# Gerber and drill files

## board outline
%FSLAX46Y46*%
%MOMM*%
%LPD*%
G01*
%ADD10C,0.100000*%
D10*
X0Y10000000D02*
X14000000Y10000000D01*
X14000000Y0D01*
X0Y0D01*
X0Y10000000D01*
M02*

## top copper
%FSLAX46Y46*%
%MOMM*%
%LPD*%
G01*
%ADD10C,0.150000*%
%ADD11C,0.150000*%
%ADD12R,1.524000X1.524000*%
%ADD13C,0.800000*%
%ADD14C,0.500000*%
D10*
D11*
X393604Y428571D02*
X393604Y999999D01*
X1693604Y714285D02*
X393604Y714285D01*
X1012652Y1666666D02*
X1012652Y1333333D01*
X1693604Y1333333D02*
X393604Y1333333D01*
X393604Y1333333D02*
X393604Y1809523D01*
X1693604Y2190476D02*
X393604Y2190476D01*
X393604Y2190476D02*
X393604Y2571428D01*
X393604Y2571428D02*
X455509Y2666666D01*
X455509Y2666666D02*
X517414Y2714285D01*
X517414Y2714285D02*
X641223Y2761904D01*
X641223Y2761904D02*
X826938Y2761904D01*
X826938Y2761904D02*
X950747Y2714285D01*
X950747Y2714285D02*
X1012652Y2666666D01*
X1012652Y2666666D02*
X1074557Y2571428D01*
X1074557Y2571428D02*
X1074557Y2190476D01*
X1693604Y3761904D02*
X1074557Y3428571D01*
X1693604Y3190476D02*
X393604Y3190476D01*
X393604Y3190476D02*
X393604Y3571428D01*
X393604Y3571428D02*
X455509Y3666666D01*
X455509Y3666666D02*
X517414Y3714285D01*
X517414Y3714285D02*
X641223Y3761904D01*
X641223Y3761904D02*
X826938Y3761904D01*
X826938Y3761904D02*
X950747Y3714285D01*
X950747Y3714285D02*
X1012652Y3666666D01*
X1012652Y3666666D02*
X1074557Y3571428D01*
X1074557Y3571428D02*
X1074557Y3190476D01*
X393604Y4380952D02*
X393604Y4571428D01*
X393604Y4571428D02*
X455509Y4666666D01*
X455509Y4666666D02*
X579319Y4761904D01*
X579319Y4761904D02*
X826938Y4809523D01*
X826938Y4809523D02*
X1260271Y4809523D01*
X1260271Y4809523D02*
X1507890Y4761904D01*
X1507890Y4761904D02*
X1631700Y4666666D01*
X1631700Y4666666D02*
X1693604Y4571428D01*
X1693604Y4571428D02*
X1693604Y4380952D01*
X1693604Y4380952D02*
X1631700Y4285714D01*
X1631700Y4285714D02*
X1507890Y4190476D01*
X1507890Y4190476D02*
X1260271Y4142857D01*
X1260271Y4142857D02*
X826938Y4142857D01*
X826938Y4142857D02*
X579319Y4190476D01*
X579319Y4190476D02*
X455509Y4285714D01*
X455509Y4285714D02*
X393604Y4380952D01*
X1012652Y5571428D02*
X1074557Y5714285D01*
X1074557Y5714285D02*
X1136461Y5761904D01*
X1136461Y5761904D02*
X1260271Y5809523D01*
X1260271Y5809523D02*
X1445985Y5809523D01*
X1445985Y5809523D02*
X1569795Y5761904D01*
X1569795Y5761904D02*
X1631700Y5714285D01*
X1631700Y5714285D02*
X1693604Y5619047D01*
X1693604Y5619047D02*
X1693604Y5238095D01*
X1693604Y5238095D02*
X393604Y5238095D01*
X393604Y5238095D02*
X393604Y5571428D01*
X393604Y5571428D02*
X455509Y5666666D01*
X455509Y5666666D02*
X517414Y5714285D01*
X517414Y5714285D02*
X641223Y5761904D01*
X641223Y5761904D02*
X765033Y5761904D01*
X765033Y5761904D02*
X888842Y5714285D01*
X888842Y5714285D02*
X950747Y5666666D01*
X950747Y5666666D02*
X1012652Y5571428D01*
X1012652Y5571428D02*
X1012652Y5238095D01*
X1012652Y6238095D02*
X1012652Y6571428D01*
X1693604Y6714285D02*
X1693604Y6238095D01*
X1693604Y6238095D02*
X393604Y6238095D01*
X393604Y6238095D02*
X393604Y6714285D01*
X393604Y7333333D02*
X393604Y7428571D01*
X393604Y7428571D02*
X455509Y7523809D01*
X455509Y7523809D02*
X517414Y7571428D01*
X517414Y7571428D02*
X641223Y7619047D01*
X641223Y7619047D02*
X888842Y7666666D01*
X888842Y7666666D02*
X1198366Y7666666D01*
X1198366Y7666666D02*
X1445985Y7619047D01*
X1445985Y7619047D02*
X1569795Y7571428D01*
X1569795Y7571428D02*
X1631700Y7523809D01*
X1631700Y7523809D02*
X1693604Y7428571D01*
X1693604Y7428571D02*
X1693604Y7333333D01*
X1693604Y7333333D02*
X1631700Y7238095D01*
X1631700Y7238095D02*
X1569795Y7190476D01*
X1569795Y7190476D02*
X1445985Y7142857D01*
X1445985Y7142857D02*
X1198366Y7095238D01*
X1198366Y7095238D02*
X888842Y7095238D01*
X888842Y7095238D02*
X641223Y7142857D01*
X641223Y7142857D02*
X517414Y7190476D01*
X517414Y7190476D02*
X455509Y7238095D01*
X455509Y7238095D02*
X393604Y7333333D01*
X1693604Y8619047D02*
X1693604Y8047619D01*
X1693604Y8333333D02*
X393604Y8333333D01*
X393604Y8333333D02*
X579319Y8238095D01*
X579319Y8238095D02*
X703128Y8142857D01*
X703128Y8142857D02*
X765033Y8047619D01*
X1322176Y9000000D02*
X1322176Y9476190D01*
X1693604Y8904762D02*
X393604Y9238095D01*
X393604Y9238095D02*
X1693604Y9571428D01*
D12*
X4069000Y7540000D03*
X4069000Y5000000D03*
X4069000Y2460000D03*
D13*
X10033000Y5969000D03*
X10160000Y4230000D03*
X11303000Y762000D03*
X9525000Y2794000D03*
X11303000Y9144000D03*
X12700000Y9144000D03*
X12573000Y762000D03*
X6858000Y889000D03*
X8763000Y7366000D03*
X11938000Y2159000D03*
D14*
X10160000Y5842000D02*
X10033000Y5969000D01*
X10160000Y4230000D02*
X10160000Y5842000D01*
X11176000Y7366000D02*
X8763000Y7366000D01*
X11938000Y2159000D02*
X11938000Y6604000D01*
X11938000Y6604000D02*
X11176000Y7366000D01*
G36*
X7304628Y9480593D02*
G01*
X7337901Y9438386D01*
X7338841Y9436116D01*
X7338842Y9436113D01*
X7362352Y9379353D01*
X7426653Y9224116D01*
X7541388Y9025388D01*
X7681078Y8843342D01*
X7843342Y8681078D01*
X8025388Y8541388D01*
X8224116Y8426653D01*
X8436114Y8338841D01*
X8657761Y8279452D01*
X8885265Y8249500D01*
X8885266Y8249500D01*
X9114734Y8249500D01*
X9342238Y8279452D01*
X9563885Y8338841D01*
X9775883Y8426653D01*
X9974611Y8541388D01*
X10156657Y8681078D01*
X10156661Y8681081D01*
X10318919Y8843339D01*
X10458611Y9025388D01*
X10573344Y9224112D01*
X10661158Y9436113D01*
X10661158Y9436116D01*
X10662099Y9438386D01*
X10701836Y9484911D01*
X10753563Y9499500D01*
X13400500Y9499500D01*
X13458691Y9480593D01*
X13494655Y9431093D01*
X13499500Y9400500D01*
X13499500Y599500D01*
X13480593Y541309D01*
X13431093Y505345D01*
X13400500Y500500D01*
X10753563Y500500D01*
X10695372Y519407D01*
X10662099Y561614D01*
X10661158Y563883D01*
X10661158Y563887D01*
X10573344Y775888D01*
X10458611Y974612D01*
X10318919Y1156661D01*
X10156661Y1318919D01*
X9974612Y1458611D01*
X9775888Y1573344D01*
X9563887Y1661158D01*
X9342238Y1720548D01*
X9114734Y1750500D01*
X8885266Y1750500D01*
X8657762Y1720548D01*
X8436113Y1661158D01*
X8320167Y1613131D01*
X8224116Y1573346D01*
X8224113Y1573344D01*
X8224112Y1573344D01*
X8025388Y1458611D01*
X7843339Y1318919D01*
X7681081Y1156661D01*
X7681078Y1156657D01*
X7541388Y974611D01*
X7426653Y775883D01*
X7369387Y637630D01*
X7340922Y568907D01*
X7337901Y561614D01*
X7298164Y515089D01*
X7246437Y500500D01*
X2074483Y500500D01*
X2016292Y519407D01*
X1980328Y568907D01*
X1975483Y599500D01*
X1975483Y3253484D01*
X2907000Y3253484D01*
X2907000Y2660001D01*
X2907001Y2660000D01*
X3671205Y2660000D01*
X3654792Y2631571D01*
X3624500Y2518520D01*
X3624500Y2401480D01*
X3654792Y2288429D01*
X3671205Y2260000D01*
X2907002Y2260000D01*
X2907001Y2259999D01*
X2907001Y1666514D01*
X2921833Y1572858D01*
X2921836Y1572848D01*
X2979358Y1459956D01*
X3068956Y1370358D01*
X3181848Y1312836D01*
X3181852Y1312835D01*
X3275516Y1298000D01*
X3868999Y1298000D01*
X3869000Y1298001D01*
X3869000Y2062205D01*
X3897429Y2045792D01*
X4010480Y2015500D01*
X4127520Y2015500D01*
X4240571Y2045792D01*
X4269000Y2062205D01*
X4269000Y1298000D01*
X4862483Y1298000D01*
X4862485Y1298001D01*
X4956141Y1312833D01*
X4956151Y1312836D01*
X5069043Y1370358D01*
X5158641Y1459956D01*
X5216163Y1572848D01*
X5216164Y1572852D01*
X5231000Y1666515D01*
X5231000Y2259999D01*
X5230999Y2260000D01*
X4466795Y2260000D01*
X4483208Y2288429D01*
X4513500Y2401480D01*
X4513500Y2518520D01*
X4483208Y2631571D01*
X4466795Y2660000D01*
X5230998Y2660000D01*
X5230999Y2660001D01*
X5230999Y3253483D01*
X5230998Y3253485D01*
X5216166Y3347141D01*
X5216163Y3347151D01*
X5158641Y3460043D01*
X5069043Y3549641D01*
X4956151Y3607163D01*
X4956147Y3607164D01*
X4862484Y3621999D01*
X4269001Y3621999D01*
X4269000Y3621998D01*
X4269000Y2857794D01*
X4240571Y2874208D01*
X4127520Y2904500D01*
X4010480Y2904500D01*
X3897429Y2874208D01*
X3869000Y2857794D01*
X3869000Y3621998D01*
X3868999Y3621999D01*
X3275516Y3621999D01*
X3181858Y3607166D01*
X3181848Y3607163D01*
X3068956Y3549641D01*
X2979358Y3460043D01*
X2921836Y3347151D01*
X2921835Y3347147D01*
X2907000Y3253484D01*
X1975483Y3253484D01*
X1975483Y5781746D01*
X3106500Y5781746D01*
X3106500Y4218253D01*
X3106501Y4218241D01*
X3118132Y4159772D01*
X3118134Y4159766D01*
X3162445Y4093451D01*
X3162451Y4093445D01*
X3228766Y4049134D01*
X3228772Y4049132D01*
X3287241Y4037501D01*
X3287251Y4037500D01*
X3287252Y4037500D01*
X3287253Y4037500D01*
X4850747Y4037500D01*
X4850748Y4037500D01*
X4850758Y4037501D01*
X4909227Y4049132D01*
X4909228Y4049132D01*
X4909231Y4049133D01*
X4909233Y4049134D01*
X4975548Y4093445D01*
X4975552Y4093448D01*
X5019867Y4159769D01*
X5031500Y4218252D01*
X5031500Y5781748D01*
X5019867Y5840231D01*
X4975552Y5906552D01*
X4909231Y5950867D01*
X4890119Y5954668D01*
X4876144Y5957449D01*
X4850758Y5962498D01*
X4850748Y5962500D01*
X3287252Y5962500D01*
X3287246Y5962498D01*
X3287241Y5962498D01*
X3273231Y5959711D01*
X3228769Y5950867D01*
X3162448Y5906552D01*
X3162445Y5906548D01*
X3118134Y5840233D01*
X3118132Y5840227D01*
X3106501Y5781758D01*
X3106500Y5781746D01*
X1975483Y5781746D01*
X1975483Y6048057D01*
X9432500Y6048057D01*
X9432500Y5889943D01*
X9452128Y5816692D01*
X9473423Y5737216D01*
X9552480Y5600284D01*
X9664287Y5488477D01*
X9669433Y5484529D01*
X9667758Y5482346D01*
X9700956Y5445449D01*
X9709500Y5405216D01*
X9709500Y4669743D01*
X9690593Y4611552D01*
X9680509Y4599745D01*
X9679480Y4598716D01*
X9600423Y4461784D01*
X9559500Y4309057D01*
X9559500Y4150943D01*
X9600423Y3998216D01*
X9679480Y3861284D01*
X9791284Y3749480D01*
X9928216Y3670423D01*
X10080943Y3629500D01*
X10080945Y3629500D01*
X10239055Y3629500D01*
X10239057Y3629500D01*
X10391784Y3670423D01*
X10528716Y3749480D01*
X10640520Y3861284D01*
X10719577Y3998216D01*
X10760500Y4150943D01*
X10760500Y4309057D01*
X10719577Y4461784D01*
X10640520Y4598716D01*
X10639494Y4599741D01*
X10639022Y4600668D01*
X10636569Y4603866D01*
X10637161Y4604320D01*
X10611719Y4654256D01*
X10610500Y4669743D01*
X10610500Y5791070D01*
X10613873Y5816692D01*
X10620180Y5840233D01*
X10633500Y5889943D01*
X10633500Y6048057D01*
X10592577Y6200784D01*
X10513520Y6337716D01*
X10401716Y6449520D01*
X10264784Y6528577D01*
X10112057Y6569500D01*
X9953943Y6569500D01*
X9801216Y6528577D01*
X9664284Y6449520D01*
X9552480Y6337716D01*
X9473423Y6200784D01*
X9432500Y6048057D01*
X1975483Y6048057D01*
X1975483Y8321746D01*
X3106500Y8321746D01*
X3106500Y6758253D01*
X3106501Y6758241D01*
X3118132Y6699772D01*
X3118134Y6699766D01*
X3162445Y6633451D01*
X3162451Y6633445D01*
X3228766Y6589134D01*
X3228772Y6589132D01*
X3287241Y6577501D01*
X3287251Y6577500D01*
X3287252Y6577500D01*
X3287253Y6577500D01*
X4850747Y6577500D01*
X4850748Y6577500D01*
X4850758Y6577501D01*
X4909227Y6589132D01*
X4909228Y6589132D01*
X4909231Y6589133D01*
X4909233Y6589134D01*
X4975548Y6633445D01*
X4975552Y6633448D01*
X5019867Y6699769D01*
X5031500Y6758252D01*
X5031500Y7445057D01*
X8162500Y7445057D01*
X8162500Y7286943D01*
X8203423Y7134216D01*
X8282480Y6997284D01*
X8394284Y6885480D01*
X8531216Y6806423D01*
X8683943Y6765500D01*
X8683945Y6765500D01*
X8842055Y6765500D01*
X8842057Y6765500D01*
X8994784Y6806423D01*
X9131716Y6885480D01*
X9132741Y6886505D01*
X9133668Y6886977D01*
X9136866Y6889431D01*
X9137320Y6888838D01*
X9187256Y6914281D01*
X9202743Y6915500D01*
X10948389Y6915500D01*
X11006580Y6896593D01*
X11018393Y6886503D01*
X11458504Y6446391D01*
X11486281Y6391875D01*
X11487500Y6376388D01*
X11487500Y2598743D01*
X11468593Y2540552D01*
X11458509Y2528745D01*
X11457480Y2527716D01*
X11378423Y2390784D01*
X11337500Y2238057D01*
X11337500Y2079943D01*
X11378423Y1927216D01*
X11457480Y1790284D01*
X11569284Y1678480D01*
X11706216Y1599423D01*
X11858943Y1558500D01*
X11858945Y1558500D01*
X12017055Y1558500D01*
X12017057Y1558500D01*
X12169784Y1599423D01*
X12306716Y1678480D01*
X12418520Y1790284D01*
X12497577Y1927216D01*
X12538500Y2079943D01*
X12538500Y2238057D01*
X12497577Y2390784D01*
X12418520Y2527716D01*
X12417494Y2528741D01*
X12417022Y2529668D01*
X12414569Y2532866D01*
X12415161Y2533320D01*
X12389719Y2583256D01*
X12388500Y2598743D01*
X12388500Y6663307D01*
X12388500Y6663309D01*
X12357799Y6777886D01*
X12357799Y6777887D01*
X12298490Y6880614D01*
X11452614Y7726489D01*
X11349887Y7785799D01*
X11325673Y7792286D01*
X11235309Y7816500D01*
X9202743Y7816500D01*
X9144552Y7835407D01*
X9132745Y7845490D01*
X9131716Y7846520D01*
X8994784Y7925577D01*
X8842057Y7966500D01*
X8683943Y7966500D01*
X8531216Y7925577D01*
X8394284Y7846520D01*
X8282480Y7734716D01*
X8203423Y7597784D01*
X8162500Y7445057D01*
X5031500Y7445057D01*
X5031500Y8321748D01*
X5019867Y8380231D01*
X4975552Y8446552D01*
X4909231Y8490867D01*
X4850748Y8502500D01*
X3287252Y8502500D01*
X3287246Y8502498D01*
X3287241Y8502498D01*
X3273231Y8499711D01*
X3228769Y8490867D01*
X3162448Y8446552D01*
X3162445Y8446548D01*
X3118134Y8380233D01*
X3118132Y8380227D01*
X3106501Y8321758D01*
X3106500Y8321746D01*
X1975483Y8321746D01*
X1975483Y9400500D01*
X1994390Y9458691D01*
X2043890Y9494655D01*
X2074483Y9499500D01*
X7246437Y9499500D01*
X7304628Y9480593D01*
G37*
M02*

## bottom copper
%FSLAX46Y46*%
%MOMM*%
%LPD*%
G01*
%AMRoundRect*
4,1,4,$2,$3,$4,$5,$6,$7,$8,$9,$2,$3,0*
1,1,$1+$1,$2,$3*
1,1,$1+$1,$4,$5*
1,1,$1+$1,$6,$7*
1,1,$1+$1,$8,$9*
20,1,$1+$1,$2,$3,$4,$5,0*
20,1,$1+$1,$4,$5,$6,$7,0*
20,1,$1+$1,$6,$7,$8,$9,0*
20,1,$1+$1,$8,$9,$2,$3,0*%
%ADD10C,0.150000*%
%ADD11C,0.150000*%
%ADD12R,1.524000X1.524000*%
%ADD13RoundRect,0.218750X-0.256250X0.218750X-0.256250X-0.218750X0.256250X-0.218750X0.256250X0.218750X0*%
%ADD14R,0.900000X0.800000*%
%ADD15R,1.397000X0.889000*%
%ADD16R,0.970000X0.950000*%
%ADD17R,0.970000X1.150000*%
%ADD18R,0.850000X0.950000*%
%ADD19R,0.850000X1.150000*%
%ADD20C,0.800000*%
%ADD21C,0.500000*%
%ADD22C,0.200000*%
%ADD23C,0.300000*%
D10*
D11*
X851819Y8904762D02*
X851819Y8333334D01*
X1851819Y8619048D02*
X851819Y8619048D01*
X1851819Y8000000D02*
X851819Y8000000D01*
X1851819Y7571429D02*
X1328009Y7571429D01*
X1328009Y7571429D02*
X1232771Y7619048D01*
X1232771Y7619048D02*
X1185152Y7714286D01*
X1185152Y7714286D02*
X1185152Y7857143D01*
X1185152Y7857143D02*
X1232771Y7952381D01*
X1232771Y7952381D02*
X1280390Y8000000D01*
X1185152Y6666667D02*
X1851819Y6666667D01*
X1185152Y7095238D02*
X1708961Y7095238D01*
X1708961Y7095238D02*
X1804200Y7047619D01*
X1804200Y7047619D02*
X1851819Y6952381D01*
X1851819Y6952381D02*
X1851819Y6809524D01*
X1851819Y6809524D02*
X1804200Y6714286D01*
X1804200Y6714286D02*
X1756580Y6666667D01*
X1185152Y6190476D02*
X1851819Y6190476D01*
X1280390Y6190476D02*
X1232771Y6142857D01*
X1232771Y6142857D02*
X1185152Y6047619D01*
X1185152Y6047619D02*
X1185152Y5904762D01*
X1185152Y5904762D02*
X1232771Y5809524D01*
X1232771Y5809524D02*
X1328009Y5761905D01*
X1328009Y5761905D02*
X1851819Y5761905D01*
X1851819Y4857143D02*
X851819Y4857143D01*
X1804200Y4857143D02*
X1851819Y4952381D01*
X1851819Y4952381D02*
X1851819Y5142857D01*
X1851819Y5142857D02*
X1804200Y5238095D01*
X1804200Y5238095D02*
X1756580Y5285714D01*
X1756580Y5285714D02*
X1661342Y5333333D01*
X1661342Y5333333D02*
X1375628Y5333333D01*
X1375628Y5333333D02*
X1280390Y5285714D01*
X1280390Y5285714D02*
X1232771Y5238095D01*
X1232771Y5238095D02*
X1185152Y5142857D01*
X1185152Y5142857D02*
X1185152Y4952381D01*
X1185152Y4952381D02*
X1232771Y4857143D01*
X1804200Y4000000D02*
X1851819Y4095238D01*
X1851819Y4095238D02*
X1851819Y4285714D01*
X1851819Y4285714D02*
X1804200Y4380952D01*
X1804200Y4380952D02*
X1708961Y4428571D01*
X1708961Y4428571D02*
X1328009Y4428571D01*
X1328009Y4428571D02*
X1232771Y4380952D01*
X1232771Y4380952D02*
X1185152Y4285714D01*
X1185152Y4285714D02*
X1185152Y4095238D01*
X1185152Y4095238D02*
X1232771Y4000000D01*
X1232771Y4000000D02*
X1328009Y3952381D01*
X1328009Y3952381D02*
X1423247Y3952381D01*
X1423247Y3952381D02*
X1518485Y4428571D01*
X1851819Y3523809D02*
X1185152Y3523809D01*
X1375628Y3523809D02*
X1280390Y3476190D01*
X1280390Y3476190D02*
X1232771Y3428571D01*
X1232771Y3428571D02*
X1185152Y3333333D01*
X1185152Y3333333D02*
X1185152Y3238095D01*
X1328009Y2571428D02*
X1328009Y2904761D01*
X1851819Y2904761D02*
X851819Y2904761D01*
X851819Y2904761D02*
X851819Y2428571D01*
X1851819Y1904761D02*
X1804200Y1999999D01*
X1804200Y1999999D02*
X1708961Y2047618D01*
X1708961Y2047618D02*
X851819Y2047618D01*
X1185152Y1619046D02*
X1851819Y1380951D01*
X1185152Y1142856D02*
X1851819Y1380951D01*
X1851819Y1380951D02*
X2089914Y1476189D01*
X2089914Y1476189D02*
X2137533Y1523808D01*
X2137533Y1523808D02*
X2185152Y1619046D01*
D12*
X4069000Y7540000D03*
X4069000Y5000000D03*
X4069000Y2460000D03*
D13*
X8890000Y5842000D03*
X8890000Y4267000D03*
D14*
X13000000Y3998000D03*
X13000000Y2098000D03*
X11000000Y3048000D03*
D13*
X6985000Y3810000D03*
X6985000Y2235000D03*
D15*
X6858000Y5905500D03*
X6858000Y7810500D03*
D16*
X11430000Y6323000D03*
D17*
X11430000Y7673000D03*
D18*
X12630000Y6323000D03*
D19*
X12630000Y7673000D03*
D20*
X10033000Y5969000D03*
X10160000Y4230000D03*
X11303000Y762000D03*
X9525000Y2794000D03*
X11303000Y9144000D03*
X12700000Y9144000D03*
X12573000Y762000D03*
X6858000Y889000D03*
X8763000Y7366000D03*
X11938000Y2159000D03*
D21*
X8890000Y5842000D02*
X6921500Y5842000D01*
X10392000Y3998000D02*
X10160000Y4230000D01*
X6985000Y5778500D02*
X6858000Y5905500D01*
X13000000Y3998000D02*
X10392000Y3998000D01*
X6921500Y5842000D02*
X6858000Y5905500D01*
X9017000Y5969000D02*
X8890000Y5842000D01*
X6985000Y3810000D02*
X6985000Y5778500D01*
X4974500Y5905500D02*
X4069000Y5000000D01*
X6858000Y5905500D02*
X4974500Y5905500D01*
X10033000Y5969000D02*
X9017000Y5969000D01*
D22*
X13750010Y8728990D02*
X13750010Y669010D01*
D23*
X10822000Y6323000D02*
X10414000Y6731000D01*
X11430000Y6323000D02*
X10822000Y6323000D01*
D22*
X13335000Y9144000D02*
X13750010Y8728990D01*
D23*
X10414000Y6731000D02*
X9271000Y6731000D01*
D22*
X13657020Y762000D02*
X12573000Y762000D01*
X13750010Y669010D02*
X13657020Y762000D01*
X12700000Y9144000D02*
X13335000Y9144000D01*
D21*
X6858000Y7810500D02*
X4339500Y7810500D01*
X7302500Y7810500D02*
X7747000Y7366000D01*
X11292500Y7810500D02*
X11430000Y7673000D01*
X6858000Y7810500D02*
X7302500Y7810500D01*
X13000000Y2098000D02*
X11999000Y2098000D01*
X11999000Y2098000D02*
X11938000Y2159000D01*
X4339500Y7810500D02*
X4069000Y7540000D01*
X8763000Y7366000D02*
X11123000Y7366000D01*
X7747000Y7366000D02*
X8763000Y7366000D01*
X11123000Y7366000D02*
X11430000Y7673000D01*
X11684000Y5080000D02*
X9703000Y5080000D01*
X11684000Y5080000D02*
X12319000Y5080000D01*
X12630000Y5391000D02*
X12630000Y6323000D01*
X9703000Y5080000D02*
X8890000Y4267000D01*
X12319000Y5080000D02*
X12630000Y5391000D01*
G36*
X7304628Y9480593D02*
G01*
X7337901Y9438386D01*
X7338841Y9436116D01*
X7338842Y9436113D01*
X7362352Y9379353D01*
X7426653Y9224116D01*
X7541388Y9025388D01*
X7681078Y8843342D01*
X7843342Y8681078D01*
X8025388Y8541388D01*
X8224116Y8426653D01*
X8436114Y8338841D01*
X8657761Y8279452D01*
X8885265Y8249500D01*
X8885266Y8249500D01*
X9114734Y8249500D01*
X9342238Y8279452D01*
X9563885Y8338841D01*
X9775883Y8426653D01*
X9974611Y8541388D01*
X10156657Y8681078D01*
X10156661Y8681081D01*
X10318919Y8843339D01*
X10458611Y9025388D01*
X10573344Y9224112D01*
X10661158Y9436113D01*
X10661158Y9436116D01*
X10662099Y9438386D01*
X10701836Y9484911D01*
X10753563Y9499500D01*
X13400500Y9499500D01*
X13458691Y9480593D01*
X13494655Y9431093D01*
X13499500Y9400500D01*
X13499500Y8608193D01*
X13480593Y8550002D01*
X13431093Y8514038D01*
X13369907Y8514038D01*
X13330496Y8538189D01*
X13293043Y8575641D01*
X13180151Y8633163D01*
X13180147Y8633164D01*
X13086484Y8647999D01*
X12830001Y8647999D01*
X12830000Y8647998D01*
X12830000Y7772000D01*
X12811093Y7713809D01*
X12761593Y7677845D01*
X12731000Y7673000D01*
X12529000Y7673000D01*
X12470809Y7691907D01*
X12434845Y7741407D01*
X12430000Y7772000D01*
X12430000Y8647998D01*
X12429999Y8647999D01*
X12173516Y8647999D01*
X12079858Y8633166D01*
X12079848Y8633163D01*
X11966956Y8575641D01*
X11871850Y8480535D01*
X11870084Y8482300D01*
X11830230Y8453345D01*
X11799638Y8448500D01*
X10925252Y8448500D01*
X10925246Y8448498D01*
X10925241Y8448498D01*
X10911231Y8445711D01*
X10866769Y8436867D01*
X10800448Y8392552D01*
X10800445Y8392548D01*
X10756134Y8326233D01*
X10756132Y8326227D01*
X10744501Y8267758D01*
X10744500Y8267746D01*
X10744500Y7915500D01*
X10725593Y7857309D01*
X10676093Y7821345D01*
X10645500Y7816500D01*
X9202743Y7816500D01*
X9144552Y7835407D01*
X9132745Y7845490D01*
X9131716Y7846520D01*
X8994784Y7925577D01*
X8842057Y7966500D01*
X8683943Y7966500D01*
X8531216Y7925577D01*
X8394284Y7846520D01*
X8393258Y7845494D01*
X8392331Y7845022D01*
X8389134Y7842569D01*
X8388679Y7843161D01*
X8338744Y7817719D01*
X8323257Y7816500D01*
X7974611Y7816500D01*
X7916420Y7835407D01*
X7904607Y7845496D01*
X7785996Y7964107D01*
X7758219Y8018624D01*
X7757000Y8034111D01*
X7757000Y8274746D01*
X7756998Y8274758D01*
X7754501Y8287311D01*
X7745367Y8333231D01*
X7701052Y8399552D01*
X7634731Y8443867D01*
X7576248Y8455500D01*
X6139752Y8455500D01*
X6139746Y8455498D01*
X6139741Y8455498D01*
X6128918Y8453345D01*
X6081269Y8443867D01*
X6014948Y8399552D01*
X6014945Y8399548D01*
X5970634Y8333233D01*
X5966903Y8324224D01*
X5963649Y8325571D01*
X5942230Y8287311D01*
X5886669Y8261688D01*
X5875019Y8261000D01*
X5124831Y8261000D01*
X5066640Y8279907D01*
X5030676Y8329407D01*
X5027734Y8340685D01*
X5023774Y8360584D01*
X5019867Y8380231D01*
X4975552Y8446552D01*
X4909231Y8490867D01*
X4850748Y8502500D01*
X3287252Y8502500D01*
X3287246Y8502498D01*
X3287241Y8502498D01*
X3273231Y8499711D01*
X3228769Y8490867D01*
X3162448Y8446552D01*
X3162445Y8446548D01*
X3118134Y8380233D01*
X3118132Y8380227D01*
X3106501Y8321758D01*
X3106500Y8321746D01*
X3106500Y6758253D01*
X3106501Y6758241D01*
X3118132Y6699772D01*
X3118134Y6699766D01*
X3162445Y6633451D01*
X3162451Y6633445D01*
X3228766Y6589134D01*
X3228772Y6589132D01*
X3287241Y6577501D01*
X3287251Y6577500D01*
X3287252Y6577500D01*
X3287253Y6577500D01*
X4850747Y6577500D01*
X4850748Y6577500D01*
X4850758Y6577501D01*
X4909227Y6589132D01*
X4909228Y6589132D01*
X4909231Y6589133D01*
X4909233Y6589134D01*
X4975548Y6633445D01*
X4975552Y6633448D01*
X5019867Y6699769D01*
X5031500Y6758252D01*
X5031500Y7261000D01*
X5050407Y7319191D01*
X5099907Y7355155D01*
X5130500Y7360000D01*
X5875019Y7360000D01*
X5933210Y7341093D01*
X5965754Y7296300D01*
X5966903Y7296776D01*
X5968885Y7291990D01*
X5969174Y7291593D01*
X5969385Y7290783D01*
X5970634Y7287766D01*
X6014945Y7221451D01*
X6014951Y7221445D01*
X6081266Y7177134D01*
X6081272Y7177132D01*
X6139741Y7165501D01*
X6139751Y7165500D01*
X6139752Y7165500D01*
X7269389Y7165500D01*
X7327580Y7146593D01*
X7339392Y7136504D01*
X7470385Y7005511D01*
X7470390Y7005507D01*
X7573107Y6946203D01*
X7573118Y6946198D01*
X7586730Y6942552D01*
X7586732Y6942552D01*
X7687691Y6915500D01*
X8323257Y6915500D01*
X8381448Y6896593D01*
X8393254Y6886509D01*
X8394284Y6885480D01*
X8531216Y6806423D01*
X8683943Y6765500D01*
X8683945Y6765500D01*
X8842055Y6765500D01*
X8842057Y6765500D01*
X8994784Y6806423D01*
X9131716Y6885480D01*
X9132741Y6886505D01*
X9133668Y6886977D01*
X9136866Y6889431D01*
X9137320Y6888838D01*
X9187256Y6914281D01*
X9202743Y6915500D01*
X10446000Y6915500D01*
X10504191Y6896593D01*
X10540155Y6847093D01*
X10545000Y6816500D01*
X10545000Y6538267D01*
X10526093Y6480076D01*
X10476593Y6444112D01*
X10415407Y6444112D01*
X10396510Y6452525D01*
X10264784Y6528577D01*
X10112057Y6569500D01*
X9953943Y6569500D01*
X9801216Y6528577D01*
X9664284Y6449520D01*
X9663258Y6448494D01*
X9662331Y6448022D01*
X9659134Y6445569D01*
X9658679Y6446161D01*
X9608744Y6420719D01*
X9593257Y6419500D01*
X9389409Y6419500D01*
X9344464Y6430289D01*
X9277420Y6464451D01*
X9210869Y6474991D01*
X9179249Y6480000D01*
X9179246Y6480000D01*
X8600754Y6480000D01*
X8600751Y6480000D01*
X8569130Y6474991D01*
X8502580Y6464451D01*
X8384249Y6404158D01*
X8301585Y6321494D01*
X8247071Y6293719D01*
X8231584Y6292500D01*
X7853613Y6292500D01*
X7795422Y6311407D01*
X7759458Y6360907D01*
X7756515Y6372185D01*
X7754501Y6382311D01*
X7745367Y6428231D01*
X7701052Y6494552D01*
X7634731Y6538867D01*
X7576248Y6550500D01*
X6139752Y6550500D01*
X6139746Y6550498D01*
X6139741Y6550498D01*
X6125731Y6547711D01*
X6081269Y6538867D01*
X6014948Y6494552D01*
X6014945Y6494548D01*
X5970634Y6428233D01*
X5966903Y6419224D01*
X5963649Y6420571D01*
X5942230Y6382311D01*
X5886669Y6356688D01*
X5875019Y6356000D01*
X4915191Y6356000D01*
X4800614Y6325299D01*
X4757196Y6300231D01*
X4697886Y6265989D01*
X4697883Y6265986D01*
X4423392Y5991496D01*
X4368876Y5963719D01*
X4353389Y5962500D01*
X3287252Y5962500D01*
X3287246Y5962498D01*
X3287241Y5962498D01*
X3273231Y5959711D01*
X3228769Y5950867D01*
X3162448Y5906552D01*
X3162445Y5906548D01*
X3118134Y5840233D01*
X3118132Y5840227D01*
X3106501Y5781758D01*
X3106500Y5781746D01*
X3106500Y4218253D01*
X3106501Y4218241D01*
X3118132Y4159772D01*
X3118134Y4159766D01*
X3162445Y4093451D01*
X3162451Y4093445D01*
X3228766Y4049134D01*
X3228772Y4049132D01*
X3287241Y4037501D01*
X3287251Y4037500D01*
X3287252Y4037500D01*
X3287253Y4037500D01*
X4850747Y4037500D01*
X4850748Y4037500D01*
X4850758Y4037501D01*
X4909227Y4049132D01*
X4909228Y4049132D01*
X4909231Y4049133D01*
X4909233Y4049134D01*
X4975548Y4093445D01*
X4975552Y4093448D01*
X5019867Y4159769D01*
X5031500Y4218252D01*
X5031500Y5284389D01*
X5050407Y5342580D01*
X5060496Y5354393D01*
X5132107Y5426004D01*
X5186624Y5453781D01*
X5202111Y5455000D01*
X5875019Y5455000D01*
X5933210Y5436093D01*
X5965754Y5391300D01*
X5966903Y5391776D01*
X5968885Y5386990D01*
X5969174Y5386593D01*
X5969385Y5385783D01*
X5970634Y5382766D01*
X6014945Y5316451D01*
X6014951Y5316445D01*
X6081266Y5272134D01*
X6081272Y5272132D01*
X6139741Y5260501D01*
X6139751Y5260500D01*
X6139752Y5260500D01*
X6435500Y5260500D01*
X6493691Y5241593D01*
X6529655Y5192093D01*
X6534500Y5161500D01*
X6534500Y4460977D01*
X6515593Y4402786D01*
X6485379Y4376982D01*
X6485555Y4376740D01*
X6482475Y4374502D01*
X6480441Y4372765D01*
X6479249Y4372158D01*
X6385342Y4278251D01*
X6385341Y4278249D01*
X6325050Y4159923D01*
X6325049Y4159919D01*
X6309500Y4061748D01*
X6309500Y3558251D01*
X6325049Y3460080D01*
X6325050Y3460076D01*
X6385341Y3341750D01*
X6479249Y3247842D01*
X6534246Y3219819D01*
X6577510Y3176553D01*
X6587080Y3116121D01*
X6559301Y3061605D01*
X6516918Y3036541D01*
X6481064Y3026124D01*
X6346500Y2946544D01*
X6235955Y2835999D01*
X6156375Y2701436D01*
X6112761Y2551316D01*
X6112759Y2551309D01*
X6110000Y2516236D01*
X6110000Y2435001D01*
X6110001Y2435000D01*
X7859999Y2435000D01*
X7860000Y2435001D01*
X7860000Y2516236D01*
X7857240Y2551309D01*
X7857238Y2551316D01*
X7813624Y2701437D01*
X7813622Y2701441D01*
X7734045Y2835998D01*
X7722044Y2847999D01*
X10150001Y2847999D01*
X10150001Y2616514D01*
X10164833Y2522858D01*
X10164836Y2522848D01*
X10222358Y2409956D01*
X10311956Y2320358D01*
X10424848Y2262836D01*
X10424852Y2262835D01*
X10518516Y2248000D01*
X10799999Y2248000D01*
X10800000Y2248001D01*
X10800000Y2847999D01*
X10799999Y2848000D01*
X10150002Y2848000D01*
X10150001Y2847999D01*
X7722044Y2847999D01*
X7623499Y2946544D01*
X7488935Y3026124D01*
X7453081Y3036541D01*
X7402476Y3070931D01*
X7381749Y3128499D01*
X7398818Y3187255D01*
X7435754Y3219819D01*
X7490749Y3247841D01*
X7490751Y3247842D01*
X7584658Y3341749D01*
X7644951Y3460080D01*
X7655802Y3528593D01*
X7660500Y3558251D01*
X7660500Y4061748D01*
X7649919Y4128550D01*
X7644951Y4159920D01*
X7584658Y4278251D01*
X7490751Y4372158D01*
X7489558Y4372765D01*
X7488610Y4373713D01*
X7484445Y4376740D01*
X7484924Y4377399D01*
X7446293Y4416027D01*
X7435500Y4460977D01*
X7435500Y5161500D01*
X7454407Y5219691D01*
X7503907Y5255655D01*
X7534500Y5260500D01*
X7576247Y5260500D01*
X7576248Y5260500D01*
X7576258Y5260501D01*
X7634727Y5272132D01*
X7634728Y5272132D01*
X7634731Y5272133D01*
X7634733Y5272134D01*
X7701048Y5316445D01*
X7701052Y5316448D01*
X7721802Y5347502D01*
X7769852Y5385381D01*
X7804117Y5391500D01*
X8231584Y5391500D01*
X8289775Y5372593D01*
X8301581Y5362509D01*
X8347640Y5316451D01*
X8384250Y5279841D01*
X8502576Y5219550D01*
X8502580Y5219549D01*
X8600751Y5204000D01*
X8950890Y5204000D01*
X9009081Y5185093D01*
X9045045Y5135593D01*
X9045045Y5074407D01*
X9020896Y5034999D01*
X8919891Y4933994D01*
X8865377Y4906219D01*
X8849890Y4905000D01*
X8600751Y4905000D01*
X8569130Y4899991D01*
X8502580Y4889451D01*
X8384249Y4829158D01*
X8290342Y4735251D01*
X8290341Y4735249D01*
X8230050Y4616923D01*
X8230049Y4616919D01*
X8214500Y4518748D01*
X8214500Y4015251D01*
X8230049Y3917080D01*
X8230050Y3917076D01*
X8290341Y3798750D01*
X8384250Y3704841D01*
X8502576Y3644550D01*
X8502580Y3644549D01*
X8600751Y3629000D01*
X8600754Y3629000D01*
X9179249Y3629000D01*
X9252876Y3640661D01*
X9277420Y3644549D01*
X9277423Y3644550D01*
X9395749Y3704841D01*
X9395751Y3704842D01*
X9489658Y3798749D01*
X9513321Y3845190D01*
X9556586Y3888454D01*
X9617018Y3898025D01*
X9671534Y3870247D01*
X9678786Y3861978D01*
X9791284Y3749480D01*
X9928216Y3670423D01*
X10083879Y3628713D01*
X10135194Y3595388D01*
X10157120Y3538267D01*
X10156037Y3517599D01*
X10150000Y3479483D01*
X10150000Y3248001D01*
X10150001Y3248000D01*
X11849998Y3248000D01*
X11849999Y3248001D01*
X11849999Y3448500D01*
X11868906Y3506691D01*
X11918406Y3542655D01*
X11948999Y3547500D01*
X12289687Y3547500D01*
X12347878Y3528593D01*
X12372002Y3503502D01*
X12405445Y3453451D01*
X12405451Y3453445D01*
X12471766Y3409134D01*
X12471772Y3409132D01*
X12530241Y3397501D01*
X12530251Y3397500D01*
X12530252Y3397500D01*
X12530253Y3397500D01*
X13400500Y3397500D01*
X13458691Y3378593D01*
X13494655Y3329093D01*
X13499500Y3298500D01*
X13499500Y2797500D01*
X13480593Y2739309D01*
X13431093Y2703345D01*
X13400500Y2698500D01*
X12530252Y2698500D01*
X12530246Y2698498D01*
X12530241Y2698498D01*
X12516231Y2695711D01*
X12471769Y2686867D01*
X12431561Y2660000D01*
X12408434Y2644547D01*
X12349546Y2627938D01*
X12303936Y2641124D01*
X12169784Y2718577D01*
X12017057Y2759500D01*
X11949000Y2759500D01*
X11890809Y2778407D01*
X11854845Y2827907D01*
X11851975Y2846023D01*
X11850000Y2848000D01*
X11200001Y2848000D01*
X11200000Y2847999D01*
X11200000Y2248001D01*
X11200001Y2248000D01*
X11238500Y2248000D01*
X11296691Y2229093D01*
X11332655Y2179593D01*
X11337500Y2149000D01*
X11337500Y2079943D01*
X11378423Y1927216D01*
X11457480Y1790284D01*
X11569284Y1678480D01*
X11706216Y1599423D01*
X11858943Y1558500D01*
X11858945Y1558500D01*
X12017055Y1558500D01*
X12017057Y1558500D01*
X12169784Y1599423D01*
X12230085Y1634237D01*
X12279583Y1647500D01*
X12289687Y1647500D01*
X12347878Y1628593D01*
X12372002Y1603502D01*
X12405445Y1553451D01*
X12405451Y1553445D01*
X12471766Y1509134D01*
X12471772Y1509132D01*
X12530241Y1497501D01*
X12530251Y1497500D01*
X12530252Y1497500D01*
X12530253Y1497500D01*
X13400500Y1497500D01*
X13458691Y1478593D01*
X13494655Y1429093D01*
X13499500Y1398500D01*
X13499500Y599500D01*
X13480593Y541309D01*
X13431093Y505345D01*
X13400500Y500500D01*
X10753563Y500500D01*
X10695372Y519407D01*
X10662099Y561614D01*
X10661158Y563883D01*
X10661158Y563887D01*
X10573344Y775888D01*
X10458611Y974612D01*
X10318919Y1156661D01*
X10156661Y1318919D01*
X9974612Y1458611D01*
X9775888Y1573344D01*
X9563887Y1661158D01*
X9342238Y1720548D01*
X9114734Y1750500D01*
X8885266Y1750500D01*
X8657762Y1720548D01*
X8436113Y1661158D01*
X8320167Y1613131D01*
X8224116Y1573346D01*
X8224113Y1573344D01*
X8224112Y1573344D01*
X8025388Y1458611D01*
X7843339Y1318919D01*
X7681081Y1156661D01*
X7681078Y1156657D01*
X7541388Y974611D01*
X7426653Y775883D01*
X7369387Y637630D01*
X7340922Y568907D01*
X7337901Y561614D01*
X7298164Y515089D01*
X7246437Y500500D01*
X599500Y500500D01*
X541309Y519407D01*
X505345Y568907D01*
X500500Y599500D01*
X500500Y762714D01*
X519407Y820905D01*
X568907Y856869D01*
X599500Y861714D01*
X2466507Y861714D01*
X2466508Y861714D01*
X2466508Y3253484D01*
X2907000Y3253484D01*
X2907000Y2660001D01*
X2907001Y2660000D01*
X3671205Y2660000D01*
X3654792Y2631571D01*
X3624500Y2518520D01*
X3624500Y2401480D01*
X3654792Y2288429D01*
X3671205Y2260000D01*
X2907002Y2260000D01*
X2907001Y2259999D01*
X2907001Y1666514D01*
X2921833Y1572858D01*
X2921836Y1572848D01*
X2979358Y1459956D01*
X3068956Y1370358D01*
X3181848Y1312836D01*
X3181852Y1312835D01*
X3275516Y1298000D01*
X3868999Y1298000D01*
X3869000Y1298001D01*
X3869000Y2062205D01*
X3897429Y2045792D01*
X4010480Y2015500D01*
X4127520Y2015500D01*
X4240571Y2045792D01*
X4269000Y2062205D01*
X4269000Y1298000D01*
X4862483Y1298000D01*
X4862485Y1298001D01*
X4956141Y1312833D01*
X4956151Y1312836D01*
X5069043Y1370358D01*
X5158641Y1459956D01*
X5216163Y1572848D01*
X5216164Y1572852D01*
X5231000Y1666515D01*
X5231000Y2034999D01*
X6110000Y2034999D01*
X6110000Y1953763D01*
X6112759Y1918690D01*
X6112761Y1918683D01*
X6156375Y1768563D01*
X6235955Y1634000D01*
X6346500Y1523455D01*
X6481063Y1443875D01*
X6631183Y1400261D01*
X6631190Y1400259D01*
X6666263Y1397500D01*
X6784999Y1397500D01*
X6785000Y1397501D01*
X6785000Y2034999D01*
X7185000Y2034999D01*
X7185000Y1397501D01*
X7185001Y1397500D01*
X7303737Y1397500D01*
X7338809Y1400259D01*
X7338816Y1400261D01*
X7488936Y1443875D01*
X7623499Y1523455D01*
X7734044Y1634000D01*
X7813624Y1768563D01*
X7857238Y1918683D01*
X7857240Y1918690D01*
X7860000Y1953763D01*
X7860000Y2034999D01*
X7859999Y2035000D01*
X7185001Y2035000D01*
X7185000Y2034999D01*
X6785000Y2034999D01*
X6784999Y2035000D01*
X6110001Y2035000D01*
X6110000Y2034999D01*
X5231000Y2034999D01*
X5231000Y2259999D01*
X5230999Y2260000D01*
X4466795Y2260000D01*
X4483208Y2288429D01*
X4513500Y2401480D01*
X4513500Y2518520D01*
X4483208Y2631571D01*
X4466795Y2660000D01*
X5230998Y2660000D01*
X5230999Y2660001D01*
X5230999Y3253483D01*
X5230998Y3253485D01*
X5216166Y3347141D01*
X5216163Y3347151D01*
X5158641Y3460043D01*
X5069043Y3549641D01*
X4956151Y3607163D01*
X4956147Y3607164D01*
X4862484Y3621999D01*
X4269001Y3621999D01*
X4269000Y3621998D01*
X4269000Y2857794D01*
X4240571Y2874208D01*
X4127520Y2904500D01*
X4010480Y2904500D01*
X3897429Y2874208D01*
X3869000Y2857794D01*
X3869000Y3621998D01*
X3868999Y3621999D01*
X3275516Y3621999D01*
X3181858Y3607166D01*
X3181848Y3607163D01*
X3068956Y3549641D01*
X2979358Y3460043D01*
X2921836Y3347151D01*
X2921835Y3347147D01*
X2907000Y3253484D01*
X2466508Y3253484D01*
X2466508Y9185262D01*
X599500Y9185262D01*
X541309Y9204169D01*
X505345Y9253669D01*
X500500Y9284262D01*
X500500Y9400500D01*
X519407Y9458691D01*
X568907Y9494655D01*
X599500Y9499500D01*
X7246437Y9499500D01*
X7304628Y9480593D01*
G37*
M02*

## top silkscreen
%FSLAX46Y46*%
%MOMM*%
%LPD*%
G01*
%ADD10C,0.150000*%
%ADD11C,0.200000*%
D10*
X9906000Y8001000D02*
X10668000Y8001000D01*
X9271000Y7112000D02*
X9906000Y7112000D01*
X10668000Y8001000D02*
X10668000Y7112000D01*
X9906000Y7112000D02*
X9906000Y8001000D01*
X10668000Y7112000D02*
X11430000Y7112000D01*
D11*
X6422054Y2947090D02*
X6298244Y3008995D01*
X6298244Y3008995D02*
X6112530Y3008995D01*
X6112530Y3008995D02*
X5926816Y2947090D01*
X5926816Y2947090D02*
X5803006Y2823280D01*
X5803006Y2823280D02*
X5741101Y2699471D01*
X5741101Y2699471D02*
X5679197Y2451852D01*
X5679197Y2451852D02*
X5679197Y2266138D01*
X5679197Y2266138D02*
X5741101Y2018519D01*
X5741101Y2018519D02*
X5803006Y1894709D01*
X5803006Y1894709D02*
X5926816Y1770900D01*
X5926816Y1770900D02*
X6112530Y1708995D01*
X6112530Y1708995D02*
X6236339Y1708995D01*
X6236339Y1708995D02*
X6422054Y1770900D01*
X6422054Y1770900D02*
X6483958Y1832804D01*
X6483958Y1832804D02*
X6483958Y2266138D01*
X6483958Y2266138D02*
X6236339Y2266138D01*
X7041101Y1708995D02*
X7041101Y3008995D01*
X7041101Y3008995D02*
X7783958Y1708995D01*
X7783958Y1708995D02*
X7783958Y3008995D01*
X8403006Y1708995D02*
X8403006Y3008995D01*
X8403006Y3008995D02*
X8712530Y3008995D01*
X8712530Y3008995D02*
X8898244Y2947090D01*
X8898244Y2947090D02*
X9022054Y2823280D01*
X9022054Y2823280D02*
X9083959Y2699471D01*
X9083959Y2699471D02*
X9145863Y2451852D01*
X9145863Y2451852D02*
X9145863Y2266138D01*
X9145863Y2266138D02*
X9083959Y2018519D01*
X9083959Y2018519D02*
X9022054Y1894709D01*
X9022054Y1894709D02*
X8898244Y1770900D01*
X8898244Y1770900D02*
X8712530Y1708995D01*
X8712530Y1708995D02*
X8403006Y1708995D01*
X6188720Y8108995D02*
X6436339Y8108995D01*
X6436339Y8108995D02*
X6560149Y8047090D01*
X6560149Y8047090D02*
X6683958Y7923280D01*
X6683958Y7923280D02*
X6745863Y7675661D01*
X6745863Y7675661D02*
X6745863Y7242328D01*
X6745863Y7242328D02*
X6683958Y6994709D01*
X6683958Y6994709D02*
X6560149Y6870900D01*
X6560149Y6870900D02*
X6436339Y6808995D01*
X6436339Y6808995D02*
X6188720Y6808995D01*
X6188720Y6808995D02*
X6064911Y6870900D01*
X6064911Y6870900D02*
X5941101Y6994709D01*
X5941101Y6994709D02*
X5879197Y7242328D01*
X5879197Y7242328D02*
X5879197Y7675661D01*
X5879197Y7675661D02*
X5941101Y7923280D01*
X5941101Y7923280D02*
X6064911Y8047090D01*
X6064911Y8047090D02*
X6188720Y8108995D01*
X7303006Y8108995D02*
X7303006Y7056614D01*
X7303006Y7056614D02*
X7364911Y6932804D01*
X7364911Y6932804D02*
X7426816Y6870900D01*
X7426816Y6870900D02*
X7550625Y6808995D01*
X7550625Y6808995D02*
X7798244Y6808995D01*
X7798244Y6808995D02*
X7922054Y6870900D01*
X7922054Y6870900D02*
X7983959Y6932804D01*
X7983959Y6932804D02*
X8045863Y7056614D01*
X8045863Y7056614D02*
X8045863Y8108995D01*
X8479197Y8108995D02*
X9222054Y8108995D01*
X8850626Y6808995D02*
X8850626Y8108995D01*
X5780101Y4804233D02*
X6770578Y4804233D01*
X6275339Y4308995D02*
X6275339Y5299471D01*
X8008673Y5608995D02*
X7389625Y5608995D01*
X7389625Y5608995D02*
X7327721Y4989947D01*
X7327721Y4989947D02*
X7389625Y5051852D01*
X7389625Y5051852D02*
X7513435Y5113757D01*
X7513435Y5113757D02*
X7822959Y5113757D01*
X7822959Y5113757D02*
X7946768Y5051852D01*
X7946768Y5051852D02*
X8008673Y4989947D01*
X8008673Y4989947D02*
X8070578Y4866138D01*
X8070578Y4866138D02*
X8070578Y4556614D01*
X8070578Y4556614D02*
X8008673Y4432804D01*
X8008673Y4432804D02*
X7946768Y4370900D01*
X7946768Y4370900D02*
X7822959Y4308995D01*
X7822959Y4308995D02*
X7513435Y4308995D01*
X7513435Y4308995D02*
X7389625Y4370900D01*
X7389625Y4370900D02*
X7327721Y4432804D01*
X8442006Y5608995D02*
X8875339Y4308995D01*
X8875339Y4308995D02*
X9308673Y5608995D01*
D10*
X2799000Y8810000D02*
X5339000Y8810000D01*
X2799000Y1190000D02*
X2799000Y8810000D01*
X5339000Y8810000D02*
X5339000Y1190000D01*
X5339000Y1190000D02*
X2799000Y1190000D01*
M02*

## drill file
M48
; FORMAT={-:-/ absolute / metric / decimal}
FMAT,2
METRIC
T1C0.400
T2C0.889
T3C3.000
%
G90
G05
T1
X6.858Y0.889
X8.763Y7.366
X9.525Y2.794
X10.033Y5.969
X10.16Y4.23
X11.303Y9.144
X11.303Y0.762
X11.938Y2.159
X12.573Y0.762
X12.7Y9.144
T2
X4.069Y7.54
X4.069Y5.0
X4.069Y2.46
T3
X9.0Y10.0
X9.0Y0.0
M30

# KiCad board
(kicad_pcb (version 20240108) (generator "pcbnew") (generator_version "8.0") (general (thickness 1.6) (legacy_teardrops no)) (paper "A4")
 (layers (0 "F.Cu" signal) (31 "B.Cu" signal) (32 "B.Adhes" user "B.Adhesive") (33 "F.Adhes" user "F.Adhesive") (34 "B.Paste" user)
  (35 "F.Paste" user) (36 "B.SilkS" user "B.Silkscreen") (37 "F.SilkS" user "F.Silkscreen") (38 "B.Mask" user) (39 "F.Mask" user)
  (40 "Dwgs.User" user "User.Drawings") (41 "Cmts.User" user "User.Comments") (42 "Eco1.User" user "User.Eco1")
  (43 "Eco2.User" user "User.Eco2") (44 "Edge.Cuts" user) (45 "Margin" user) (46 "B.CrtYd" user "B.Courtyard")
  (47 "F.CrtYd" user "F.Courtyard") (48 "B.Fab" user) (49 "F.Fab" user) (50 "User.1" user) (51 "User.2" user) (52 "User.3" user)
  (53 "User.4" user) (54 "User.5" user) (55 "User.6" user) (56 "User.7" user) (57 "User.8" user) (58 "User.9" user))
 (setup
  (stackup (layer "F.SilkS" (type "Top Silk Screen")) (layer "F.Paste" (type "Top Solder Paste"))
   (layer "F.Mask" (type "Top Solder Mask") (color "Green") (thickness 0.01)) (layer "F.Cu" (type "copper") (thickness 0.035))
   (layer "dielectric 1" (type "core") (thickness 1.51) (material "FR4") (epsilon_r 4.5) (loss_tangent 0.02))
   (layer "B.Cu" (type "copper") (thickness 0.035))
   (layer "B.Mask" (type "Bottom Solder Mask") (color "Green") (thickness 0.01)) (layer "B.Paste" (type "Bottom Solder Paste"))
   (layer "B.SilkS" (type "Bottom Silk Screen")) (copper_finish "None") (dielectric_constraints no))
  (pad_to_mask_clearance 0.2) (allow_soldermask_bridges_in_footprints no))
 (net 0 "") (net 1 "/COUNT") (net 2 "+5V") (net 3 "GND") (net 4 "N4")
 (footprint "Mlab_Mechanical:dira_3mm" (layer "F.Cu") (at 8.89 -10.033)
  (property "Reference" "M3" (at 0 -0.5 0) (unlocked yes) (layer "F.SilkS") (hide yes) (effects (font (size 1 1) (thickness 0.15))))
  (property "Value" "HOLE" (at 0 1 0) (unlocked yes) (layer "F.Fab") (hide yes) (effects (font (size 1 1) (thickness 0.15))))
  (pad "" np_thru_hole circle (at 0.11 0.033) (size 3 3) (drill 3) (layers "*.Mask")))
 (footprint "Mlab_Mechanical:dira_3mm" (layer "F.Cu") (at 9 0)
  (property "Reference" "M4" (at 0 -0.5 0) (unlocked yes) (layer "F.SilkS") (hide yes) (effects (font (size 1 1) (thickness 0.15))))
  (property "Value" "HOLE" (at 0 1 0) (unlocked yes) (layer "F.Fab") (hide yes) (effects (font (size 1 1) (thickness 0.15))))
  (pad "" np_thru_hole circle (at 0 0) (size 3 3) (drill 3) (layers "*.Mask")))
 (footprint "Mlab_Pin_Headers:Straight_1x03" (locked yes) (layer "F.Cu") (at 4.069 -5)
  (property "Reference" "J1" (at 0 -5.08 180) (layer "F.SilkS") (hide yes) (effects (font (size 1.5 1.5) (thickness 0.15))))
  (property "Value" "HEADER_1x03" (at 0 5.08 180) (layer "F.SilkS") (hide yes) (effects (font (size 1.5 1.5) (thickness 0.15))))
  (fp_line (start -1.27 -3.81) (end 1.27 -3.81) (stroke (width 0.15) (type solid)) (layer "F.SilkS"))
  (fp_line (start -1.27 3.81) (end -1.27 -3.81) (stroke (width 0.15) (type solid)) (layer "F.SilkS"))
  (fp_line (start 1.27 -3.81) (end 1.27 3.81) (stroke (width 0.15) (type solid)) (layer "F.SilkS"))
  (fp_line (start 1.27 3.81) (end -1.27 3.81) (stroke (width 0.15) (type solid)) (layer "F.SilkS"))
  (pad "1" thru_hole rect (at 0 -2.54) (size 1.524 1.524) (drill 0.889) (layers "*.Cu" "*.Mask") (remove_unused_layers no) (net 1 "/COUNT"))
  (pad "2" thru_hole rect (at 0 0) (size 1.524 1.524) (drill 0.889) (layers "*.Cu" "*.Mask") (remove_unused_layers no) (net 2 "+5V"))
  (pad "3" thru_hole rect (at 0 2.54) (size 1.524 1.524) (drill 0.889) (layers "*.Cu" "*.Mask") (remove_unused_layers no) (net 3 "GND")))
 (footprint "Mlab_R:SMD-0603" (layer "B.Cu") (at 8.89 -5.0545 -90)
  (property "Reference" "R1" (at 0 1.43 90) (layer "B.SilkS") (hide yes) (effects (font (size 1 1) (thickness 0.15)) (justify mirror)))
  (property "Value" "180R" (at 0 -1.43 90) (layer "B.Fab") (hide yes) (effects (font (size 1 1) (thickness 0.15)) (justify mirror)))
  (pad "1" smd roundrect (at -0.7875 0 270) (size 0.875 0.95) (layers "B.Cu" "B.Paste" "B.Mask") (roundrect_rratio 0.25) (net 2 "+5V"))
  (pad "2" smd roundrect (at 0.7875 0 270) (size 0.875 0.95) (layers "B.Cu" "B.Paste" "B.Mask") (roundrect_rratio 0.25) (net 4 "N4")))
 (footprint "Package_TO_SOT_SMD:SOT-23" (layer "B.Cu") (at 12 -3.048 180)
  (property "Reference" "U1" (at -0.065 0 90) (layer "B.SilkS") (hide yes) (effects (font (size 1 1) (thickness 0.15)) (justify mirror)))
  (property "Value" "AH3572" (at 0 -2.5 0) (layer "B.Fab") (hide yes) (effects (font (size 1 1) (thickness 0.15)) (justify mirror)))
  (pad "1" smd rect (at -1 0.95 180) (size 0.9 0.8) (layers "B.Cu" "B.Paste" "B.Mask") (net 2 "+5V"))
  (pad "2" smd rect (at -1 -0.95 180) (size 0.9 0.8) (layers "B.Cu" "B.Paste" "B.Mask") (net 1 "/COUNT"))
  (pad "3" smd rect (at 1 0 180) (size 0.9 0.8) (layers "B.Cu" "B.Paste" "B.Mask") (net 3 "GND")))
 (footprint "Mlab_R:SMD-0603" (layer "B.Cu") (at 6.985 -3.0225 -90)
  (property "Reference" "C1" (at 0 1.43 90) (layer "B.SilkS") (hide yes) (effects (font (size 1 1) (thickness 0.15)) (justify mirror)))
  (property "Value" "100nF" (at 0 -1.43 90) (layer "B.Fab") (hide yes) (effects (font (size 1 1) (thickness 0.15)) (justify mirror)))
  (pad "1" smd roundrect (at -0.7875 0 270) (size 0.875 0.95) (layers "B.Cu" "B.Paste" "B.Mask") (roundrect_rratio 0.25) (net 2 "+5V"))
  (pad "2" smd roundrect (at 0.7875 0 270) (size 0.875 0.95) (layers "B.Cu" "B.Paste" "B.Mask") (roundrect_rratio 0.25) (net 3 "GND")))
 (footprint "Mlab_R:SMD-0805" (layer "B.Cu") (at 6.858 -6.858 90)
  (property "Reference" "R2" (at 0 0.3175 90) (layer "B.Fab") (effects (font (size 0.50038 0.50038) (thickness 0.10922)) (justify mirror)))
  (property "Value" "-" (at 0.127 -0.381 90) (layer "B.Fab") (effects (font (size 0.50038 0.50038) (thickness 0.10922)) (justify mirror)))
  (pad "1" smd rect (at -0.9525 0 90) (size 0.889 1.397) (layers "B.Cu" "B.Paste" "B.Mask") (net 2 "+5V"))
  (pad "2" smd rect (at 0.9525 0 90) (size 0.889 1.397) (layers "B.Cu" "B.Paste" "B.Mask") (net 1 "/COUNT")))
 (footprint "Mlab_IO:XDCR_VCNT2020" (layer "B.Cu") (at 12 -7.048)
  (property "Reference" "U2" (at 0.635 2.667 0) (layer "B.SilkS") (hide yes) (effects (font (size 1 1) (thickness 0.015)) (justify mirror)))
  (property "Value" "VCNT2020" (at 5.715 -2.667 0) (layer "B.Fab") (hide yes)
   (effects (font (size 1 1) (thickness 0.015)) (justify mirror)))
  (pad "1" smd rect (at -0.57 0.725) (size 0.97 0.95) (layers "B.Cu" "B.Paste" "B.Mask") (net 3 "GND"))
  (pad "2" smd rect (at -0.57 -0.625) (size 0.97 1.15) (layers "B.Cu" "B.Paste" "B.Mask") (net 1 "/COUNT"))
  (pad "3" smd rect (at 0.63 0.725) (size 0.85 0.95) (layers "B.Cu" "B.Paste" "B.Mask") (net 4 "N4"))
  (pad "4" smd rect (at 0.63 -0.625) (size 0.85 1.15) (layers "B.Cu" "B.Paste" "B.Mask") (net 3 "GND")))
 (gr_line (start 9.906 -8.001) (end 10.668 -8.001) (stroke (width 0.15) (type solid)) (layer "F.SilkS"))
 (gr_line (start 9.271 -7.112) (end 9.906 -7.112) (stroke (width 0.15) (type solid)) (layer "F.SilkS"))
 (gr_line (start 10.668 -8.001) (end 10.668 -7.112) (stroke (width 0.15) (type solid)) (layer "F.SilkS"))
 (gr_line (start 9.906 -7.112) (end 9.906 -8.001) (stroke (width 0.15) (type solid)) (layer "F.SilkS"))
 (gr_line (start 10.668 -7.112) (end 11.43 -7.112) (stroke (width 0.15) (type solid)) (layer "F.SilkS"))
 (gr_rect (start 0 -10) (end 14 0) (stroke (width 0.1) (type solid)) (fill none) (layer "Edge.Cuts"))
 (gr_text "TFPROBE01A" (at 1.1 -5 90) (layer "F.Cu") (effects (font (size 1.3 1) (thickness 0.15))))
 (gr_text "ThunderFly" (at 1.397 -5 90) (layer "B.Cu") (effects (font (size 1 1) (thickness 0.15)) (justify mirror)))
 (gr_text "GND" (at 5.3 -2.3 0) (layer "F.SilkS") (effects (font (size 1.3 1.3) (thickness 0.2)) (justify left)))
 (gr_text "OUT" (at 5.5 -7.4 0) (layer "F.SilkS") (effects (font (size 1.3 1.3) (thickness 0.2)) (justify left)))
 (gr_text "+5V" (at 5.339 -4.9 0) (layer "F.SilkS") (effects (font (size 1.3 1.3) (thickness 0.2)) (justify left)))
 (segment (start 10.16 -5.842) (end 10.033 -5.969) (width 0.5) (layer "F.Cu") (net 2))
 (segment (start 10.16 -4.23) (end 10.16 -5.842) (width 0.5) (layer "F.Cu") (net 2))
 (via (at 10.033 -5.969) (size 0.8) (drill 0.4) (layers "F.Cu" "B.Cu") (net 2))
 (via (at 10.16 -4.23) (size 0.8) (drill 0.4) (layers "F.Cu" "B.Cu") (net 2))
 (segment (start 8.89 -5.842) (end 6.9215 -5.842) (width 0.5) (layer "B.Cu") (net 2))
 (segment (start 10.392 -3.998) (end 10.16 -4.23) (width 0.5) (layer "B.Cu") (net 2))
 (segment (start 6.985 -5.7785) (end 6.858 -5.9055) (width 0.5) (layer "B.Cu") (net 2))
 (segment (start 13 -3.998) (end 10.392 -3.998) (width 0.5) (layer "B.Cu") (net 2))
 (segment (start 6.9215 -5.842) (end 6.858 -5.9055) (width 0.5) (layer "B.Cu") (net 2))
 (segment (start 9.017 -5.969) (end 8.89 -5.842) (width 0.5) (layer "B.Cu") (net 2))
 (segment (start 6.985 -3.81) (end 6.985 -5.7785) (width 0.5) (layer "B.Cu") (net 2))
 (segment (start 4.9745 -5.9055) (end 4.069 -5) (width 0.5) (layer "B.Cu") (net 2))
 (segment (start 6.858 -5.9055) (end 4.9745 -5.9055) (width 0.5) (layer "B.Cu") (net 2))
 (segment (start 10.033 -5.969) (end 9.017 -5.969) (width 0.5) (layer "B.Cu") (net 2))
 (via (at 11.303 -0.762) (size 0.8) (drill 0.4) (layers "F.Cu" "B.Cu") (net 3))
 (via (at 9.525 -2.794) (size 0.8) (drill 0.4) (layers "F.Cu" "B.Cu") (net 3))
 (via (at 11.303 -9.144) (size 0.8) (drill 0.4) (layers "F.Cu" "B.Cu") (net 3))
 (via (at 12.7 -9.144) (size 0.8) (drill 0.4) (layers "F.Cu" "B.Cu") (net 3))
 (via (at 12.573 -0.762) (size 0.8) (drill 0.4) (layers "F.Cu" "B.Cu") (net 3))
 (via (at 6.858 -0.889) (size 0.8) (drill 0.4) (layers "F.Cu" "B.Cu") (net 3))
 (segment (start 13.75001 -8.72899) (end 13.75001 -0.66901) (width 0.2) (layer "B.Cu") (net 3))
 (segment (start 10.822 -6.323) (end 10.414 -6.731) (width 0.3) (layer "B.Cu") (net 3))
 (segment (start 11.43 -6.323) (end 10.822 -6.323) (width 0.3) (layer "B.Cu") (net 3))
 (segment (start 13.335 -9.144) (end 13.75001 -8.72899) (width 0.2) (layer "B.Cu") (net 3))
 (segment (start 10.414 -6.731) (end 9.271 -6.731) (width 0.3) (layer "B.Cu") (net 3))
 (segment (start 13.65702 -0.762) (end 12.573 -0.762) (width 0.2) (layer "B.Cu") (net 3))
 (segment (start 13.75001 -0.66901) (end 13.65702 -0.762) (width 0.2) (layer "B.Cu") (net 3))
 (segment (start 12.7 -9.144) (end 13.335 -9.144) (width 0.2) (layer "B.Cu") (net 3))
 (segment (start 11.176 -7.366) (end 8.763 -7.366) (width 0.5) (layer "F.Cu") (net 1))
 (segment (start 11.938 -2.159) (end 11.938 -6.604) (width 0.5) (layer "F.Cu") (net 1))
 (segment (start 11.938 -6.604) (end 11.176 -7.366) (width 0.5) (layer "F.Cu") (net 1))
 (via (at 8.763 -7.366) (size 0.8) (drill 0.4) (layers "F.Cu" "B.Cu") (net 1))
 (via (at 11.938 -2.159) (size 0.8) (drill 0.4) (layers "F.Cu" "B.Cu") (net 1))
 (segment (start 6.858 -7.8105) (end 4.3395 -7.8105) (width 0.5) (layer "B.Cu") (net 1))
 (segment (start 7.3025 -7.8105) (end 7.747 -7.366) (width 0.5) (layer "B.Cu") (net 1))
 (segment (start 11.2925 -7.8105) (end 11.43 -7.673) (width 0.5) (layer "B.Cu") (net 1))
 (segment (start 6.858 -7.8105) (end 7.3025 -7.8105) (width 0.5) (layer "B.Cu") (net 1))
 (segment (start 13 -2.098) (end 11.999 -2.098) (width 0.5) (layer "B.Cu") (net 1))
 (segment (start 11.999 -2.098) (end 11.938 -2.159) (width 0.5) (layer "B.Cu") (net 1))
 (segment (start 4.3395 -7.8105) (end 4.069 -7.54) (width 0.5) (layer "B.Cu") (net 1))
 (segment (start 8.763 -7.366) (end 11.123 -7.366) (width 0.5) (layer "B.Cu") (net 1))
 (segment (start 7.747 -7.366) (end 8.763 -7.366) (width 0.5) (layer "B.Cu") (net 1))
 (segment (start 11.123 -7.366) (end 11.43 -7.673) (width 0.5) (layer "B.Cu") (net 1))
 (segment (start 11.684 -5.08) (end 9.703 -5.08) (width 0.5) (layer "B.Cu") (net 4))
 (segment (start 11.684 -5.08) (end 12.319 -5.08) (width 0.5) (layer "B.Cu") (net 4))
 (segment (start 12.63 -5.391) (end 12.63 -6.323) (width 0.5) (layer "B.Cu") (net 4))
 (segment (start 9.703 -5.08) (end 8.89 -4.267) (width 0.5) (layer "B.Cu") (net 4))
 (segment (start 12.319 -5.08) (end 12.63 -5.391) (width 0.5) (layer "B.Cu") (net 4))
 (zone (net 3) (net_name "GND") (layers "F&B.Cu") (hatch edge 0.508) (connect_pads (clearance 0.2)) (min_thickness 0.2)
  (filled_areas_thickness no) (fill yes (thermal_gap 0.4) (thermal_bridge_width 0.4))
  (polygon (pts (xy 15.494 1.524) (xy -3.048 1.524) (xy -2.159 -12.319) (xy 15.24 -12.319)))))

